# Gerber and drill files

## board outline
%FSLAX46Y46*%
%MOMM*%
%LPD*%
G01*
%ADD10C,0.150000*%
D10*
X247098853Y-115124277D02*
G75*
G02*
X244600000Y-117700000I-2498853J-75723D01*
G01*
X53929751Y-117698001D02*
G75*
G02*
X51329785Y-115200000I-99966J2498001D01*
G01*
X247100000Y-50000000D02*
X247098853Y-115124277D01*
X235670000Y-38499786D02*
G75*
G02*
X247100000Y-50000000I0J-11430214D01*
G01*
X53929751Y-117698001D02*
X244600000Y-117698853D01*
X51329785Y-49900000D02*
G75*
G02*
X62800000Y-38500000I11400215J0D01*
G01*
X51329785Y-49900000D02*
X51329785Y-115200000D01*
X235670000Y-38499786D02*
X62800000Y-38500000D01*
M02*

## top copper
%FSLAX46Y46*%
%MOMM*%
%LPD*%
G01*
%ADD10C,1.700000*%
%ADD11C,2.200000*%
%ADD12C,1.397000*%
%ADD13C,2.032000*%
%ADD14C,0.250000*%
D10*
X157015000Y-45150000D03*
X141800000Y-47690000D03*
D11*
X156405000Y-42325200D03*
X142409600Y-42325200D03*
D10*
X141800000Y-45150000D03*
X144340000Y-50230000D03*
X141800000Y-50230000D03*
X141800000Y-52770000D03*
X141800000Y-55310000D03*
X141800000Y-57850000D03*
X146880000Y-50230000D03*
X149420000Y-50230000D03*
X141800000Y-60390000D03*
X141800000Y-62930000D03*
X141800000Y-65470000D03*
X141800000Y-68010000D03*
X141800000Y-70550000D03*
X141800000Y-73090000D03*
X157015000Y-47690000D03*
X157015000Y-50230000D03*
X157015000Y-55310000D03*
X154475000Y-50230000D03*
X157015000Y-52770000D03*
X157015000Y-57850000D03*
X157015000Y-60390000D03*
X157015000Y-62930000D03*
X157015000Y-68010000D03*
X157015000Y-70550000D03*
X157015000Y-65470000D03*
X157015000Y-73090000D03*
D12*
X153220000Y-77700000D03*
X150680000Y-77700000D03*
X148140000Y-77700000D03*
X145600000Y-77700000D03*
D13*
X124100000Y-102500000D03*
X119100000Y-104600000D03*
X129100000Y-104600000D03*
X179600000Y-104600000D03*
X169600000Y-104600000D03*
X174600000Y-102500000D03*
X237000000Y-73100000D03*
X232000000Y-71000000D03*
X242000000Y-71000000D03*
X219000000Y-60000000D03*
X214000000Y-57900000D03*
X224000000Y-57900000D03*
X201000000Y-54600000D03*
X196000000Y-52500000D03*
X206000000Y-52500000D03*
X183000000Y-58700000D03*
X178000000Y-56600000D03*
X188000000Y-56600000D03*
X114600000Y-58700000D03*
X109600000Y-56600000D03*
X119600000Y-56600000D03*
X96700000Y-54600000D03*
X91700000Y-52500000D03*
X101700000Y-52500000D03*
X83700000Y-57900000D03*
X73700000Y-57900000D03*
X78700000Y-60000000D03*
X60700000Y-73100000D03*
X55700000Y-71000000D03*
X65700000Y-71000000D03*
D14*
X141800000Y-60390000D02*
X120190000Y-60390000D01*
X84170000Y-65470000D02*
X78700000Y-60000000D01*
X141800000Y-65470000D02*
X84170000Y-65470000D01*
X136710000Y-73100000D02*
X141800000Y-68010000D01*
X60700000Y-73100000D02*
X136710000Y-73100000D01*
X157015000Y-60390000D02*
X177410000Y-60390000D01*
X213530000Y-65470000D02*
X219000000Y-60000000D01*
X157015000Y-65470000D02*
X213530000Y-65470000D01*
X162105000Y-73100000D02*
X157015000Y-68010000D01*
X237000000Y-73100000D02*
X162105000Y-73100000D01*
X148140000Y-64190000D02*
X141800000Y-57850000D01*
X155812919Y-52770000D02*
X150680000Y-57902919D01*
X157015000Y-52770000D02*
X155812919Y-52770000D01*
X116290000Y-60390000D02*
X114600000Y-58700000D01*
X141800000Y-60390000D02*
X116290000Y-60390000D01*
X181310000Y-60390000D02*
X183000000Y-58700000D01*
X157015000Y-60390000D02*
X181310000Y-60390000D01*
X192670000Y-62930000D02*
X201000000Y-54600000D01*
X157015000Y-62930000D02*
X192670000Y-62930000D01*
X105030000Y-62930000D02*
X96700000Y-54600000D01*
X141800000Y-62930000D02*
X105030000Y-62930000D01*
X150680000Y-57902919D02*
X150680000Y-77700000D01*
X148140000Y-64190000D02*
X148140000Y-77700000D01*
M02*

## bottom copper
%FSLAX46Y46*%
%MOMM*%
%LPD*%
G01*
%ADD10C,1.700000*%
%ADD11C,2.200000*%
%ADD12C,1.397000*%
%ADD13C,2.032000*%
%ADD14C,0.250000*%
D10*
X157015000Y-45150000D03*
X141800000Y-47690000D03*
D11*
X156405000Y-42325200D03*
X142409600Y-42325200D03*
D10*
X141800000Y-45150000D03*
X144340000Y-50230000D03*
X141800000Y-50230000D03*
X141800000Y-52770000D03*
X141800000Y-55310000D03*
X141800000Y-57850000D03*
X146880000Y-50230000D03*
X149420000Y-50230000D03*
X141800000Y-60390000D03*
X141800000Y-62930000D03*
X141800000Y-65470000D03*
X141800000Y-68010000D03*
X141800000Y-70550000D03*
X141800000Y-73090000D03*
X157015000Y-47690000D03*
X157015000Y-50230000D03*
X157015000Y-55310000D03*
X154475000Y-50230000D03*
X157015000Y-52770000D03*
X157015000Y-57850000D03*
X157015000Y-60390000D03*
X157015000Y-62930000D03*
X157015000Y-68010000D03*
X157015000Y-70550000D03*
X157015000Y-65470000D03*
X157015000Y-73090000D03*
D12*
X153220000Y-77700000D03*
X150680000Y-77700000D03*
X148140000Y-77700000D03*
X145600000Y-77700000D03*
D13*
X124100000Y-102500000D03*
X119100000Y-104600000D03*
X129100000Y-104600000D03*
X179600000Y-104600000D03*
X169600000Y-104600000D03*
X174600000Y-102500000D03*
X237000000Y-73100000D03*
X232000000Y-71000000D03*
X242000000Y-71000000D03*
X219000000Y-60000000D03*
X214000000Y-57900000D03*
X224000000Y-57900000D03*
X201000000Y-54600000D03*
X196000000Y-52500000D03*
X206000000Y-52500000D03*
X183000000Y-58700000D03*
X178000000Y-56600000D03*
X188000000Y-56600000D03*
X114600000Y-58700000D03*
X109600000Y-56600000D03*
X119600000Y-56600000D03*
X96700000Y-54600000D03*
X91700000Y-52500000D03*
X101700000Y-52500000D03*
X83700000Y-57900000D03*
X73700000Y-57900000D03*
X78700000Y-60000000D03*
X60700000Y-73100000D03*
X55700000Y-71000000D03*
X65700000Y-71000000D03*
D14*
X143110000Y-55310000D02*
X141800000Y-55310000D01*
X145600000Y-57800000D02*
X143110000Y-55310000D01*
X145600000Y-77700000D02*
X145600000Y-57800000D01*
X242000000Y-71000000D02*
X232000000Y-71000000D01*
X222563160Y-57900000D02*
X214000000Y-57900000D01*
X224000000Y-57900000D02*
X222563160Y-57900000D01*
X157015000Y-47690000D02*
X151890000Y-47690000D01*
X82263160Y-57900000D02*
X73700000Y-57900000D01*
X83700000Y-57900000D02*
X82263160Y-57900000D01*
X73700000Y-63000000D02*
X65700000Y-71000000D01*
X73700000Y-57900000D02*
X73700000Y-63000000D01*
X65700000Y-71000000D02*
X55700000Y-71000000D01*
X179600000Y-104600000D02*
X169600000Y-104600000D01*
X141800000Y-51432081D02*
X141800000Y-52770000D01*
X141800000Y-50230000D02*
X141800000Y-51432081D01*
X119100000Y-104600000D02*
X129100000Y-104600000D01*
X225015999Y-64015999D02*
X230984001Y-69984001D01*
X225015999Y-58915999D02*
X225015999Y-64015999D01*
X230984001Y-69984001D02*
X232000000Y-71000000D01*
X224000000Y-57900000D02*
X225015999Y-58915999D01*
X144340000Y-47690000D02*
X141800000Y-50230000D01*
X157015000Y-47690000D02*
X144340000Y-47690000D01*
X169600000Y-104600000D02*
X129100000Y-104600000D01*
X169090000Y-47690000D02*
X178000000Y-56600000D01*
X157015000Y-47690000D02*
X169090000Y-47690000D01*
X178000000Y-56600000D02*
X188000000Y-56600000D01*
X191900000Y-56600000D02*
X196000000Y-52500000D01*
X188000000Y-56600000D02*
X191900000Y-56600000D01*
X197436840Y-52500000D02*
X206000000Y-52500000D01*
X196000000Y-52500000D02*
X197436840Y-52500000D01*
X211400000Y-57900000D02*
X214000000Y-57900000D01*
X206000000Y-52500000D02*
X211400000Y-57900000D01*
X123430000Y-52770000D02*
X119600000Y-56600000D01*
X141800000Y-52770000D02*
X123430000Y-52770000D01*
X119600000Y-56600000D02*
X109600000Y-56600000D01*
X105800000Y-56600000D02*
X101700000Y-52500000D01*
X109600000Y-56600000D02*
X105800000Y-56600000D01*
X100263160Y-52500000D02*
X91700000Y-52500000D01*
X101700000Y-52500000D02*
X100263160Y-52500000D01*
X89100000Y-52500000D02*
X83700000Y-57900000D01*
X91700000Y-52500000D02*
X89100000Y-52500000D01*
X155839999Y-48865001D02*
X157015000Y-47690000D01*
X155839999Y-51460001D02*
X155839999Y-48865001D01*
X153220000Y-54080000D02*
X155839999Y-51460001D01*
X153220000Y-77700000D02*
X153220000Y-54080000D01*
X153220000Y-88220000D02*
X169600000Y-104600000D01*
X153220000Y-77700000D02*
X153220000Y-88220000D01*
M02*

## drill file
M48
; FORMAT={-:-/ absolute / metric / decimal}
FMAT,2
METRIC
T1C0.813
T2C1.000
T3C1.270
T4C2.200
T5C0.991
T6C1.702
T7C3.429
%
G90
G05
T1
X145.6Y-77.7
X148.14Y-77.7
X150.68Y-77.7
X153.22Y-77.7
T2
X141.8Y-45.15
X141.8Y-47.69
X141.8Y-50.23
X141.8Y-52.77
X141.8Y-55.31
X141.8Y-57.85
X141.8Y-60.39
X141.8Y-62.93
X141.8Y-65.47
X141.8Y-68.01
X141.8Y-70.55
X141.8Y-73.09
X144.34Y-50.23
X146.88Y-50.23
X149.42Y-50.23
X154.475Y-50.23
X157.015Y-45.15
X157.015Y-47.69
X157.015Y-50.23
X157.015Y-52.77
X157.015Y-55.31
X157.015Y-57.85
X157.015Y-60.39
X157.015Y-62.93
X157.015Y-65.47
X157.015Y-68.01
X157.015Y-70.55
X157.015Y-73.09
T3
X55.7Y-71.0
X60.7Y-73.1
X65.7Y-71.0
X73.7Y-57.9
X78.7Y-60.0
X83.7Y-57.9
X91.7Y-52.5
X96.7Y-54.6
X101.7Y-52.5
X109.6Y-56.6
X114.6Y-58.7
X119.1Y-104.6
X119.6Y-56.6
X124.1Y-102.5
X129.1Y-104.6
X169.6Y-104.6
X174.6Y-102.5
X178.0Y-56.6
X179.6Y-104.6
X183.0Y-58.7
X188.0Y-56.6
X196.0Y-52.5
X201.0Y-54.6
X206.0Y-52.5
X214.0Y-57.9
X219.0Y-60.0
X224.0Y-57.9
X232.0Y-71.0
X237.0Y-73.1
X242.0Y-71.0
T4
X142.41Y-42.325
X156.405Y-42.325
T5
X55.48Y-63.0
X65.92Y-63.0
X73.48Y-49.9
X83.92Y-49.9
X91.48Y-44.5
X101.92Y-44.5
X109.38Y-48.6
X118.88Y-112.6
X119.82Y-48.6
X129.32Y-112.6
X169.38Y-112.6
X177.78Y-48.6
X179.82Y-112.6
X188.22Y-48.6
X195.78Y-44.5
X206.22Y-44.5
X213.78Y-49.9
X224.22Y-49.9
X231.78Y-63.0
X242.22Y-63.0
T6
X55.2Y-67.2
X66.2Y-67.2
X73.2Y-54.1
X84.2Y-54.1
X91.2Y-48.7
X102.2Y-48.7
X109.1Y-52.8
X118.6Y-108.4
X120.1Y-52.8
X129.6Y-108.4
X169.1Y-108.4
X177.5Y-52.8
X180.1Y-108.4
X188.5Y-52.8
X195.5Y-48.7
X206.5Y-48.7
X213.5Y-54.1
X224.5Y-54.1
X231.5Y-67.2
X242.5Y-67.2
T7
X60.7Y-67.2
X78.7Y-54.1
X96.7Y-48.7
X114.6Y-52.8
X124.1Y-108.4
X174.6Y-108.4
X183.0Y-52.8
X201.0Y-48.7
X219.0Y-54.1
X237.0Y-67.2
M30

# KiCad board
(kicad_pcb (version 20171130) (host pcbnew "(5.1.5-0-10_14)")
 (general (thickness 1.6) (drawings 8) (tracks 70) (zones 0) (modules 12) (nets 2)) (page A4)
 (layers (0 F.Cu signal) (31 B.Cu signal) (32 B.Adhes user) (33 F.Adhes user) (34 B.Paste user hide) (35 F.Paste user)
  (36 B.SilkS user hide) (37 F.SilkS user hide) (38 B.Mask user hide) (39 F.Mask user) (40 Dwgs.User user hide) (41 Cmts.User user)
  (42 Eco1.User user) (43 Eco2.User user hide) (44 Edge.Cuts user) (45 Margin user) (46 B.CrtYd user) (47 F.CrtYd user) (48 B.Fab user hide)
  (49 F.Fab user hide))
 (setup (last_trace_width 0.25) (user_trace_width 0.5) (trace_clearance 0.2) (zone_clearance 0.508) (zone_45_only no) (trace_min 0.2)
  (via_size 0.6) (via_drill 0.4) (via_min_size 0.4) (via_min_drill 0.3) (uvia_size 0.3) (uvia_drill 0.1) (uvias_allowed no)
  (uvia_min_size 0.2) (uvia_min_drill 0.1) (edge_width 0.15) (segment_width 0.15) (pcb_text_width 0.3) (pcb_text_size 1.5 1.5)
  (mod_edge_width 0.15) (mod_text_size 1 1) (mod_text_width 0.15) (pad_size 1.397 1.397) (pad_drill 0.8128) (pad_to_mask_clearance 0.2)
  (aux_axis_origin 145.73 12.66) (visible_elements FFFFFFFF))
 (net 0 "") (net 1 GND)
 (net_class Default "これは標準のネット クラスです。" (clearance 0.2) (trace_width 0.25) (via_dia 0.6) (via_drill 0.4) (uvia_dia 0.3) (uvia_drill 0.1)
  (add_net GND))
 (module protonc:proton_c (layer F.Cu) (at 149.4 60.4)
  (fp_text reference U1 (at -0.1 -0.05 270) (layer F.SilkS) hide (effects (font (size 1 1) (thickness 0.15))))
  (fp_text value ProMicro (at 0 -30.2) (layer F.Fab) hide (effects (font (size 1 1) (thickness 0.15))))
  (pad 5V thru_hole circle (at 7.615 -15.25) (size 1.7 1.7) (drill 1) (layers *.Cu *.Mask))
  (pad A10 thru_hole circle (at -7.6 -12.71) (size 1.7 1.7) (drill 1) (layers *.Cu *.Mask))
  (pad SCRE thru_hole circle (at 7.005 -18.0748) (size 2.2 2.2) (drill 2.2) (layers *.Cu *.Mask))
  (pad SCRE thru_hole circle (at -6.9904 -18.0748) (size 2.2 2.2) (drill 2.2) (layers *.Cu *.Mask))
  (pad A9 thru_hole circle (at -7.6 -15.25) (size 1.7 1.7) (drill 1) (layers *.Cu *.Mask))
  (pad D+ thru_hole circle (at -5.06 -10.17) (size 1.7 1.7) (drill 1) (layers *.Cu *.Mask))
  (pad GND thru_hole circle (at -7.6 -10.17) (size 1.7 1.7) (drill 1) (layers *.Cu *.Mask) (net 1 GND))
  (pad GND thru_hole circle (at -7.6 -7.63) (size 1.7 1.7) (drill 1) (layers *.Cu *.Mask) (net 1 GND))
  (pad B7 thru_hole circle (at -7.6 -5.09) (size 1.7 1.7) (drill 1) (layers *.Cu *.Mask))
  (pad B6 thru_hole circle (at -7.6 -2.55) (size 1.7 1.7) (drill 1) (layers *.Cu *.Mask))
  (pad D- thru_hole circle (at -2.52 -10.17) (size 1.7 1.7) (drill 1) (layers *.Cu *.Mask))
  (pad CHRG thru_hole circle (at 0.02 -10.17) (size 1.7 1.7) (drill 1) (layers *.Cu *.Mask))
  (pad B5 thru_hole circle (at -7.6 -0.01) (size 1.7 1.7) (drill 1) (layers *.Cu *.Mask))
  (pad B4 thru_hole circle (at -7.6 2.53) (size 1.7 1.7) (drill 1) (layers *.Cu *.Mask))
  (pad B3 thru_hole circle (at -7.6 5.07) (size 1.7 1.7) (drill 1) (layers *.Cu *.Mask))
  (pad B2 thru_hole circle (at -7.6 7.61) (size 1.7 1.7) (drill 1) (layers *.Cu *.Mask))
  (pad B1 thru_hole circle (at -7.6 10.15) (size 1.7 1.7) (drill 1) (layers *.Cu *.Mask))
  (pad B0 thru_hole circle (at -7.6 12.69) (size 1.7 1.7) (drill 1) (layers *.Cu *.Mask))
  (pad GND thru_hole circle (at 7.615 -12.71) (size 1.7 1.7) (drill 1) (layers *.Cu *.Mask) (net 1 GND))
  (pad DFU thru_hole circle (at 7.615 -10.17) (size 1.7 1.7) (drill 1) (layers *.Cu *.Mask))
  (pad A2 thru_hole circle (at 7.615 -5.09) (size 1.7 1.7) (drill 1) (layers *.Cu *.Mask))
  (pad A3|5v thru_hole circle (at 5.075 -10.17) (size 1.7 1.7) (drill 1) (layers *.Cu *.Mask))
  (pad 3.3V thru_hole circle (at 7.615 -7.63) (size 1.7 1.7) (drill 1) (layers *.Cu *.Mask))
  (pad A1 thru_hole circle (at 7.615 -2.55) (size 1.7 1.7) (drill 1) (layers *.Cu *.Mask))
  (pad A0 thru_hole circle (at 7.615 -0.01) (size 1.7 1.7) (drill 1) (layers *.Cu *.Mask))
  (pad B8 thru_hole circle (at 7.615 2.53) (size 1.7 1.7) (drill 1) (layers *.Cu *.Mask))
  (pad B14 thru_hole circle (at 7.615 7.61) (size 1.7 1.7) (drill 1) (layers *.Cu *.Mask))
  (pad B15 thru_hole circle (at 7.615 10.15) (size 1.7 1.7) (drill 1) (layers *.Cu *.Mask))
  (pad B13 thru_hole circle (at 7.615 5.07) (size 1.7 1.7) (drill 1) (layers *.Cu *.Mask))
  (pad B9 thru_hole circle (at 7.615 12.69) (size 1.7 1.7) (drill 1) (layers *.Cu *.Mask)))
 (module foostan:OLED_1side (layer F.Cu) (at 145.6 77.7)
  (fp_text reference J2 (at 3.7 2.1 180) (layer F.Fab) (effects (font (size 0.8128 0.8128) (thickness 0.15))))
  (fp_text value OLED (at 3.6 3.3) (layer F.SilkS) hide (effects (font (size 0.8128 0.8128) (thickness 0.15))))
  (pad 4 thru_hole circle (at 7.62 0) (size 1.397 1.397) (drill 0.8128) (layers *.Cu F.SilkS B.Mask) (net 1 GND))
  (pad 3 thru_hole circle (at 5.08 0) (size 1.397 1.397) (drill 0.8128) (layers *.Cu F.SilkS B.Mask))
  (pad 2 thru_hole circle (at 2.54 0) (size 1.397 1.397) (drill 0.8128) (layers *.Cu F.SilkS B.Mask))
  (pad 1 thru_hole circle (at 0 0) (size 1.397 1.397) (drill 0.8128) (layers *.Cu F.SilkS B.Mask)))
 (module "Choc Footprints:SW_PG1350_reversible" (layer B.Cu) (at 124.1 108.4)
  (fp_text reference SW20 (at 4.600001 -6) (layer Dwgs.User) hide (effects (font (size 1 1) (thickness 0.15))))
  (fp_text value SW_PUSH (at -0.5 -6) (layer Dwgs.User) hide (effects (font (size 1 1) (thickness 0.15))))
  (pad "" np_thru_hole circle (at -5.5 0) (size 1.7018 1.7018) (drill 1.7018) (layers *.Cu *.Mask))
  (pad "" np_thru_hole circle (at 5.5 0) (size 1.7018 1.7018) (drill 1.7018) (layers *.Cu *.Mask))
  (pad "" np_thru_hole circle (at 5.22 4.2) (size 0.9906 0.9906) (drill 0.9906) (layers *.Cu *.Mask))
  (pad 1 thru_hole circle (at 0 -5.9) (size 2.032 2.032) (drill 1.27) (layers *.Cu *.Mask))
  (pad 2 thru_hole circle (at -5 -3.8) (size 2.032 2.032) (drill 1.27) (layers *.Cu *.Mask) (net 1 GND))
  (pad "" np_thru_hole circle (at 0 0) (size 3.429 3.429) (drill 3.429) (layers *.Cu *.Mask))
  (pad 2 thru_hole circle (at 5 -3.8) (size 2.032 2.032) (drill 1.27) (layers *.Cu *.Mask) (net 1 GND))
  (pad "" np_thru_hole circle (at -5.22 4.2) (size 0.9906 0.9906) (drill 0.9906) (layers *.Cu *.Mask)))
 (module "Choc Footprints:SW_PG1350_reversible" (layer B.Cu) (at 174.6 108.4)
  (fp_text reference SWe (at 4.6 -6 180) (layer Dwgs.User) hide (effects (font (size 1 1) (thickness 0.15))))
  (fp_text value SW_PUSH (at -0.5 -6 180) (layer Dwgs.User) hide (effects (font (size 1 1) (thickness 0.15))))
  (pad "" np_thru_hole circle (at -5.22 4.2) (size 0.9906 0.9906) (drill 0.9906) (layers *.Cu *.Mask))
  (pad 2 thru_hole circle (at 5 -3.8) (size 2.032 2.032) (drill 1.27) (layers *.Cu *.Mask) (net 1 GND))
  (pad "" np_thru_hole circle (at 0 0) (size 3.429 3.429) (drill 3.429) (layers *.Cu *.Mask))
  (pad 2 thru_hole circle (at -5 -3.8) (size 2.032 2.032) (drill 1.27) (layers *.Cu *.Mask) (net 1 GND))
  (pad 1 thru_hole circle (at 0 -5.9) (size 2.032 2.032) (drill 1.27) (layers *.Cu *.Mask))
  (pad "" np_thru_hole circle (at 5.22 4.2) (size 0.9906 0.9906) (drill 0.9906) (layers *.Cu *.Mask))
  (pad "" np_thru_hole circle (at 5.5 0) (size 1.7018 1.7018) (drill 1.7018) (layers *.Cu *.Mask))
  (pad "" np_thru_hole circle (at -5.5 0) (size 1.7018 1.7018) (drill 1.7018) (layers *.Cu *.Mask)))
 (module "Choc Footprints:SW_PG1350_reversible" (layer F.Cu) (at 237 67.2)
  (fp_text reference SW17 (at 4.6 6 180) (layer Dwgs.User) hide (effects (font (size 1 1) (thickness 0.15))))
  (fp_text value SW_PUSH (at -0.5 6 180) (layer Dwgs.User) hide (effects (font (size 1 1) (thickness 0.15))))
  (pad "" np_thru_hole circle (at -5.5 0) (size 1.7018 1.7018) (drill 1.7018) (layers *.Cu *.Mask))
  (pad "" np_thru_hole circle (at 5.5 0) (size 1.7018 1.7018) (drill 1.7018) (layers *.Cu *.Mask))
  (pad "" np_thru_hole circle (at 5.22 -4.2) (size 0.9906 0.9906) (drill 0.9906) (layers *.Cu *.Mask))
  (pad 1 thru_hole circle (at 0 5.9) (size 2.032 2.032) (drill 1.27) (layers *.Cu *.Mask))
  (pad 2 thru_hole circle (at -5 3.8) (size 2.032 2.032) (drill 1.27) (layers *.Cu *.Mask) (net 1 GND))
  (pad "" np_thru_hole circle (at 0 0) (size 3.429 3.429) (drill 3.429) (layers *.Cu *.Mask))
  (pad 2 thru_hole circle (at 5 3.8) (size 2.032 2.032) (drill 1.27) (layers *.Cu *.Mask) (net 1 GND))
  (pad "" np_thru_hole circle (at -5.22 -4.2) (size 0.9906 0.9906) (drill 0.9906) (layers *.Cu *.Mask)))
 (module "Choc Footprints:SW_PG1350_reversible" (layer F.Cu) (at 219 54.1)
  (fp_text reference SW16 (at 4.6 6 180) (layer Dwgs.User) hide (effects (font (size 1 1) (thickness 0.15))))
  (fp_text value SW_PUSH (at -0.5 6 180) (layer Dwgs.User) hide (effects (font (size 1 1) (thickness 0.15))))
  (pad "" np_thru_hole circle (at -5.5 0) (size 1.7018 1.7018) (drill 1.7018) (layers *.Cu *.Mask))
  (pad "" np_thru_hole circle (at 5.5 0) (size 1.7018 1.7018) (drill 1.7018) (layers *.Cu *.Mask))
  (pad "" np_thru_hole circle (at 5.22 -4.2) (size 0.9906 0.9906) (drill 0.9906) (layers *.Cu *.Mask))
  (pad 1 thru_hole circle (at 0 5.9) (size 2.032 2.032) (drill 1.27) (layers *.Cu *.Mask))
  (pad 2 thru_hole circle (at -5 3.8) (size 2.032 2.032) (drill 1.27) (layers *.Cu *.Mask) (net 1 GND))
  (pad "" np_thru_hole circle (at 0 0) (size 3.429 3.429) (drill 3.429) (layers *.Cu *.Mask))
  (pad 2 thru_hole circle (at 5 3.8) (size 2.032 2.032) (drill 1.27) (layers *.Cu *.Mask) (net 1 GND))
  (pad "" np_thru_hole circle (at -5.22 -4.2) (size 0.9906 0.9906) (drill 0.9906) (layers *.Cu *.Mask)))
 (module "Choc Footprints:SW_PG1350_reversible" (layer F.Cu) (at 201 48.7)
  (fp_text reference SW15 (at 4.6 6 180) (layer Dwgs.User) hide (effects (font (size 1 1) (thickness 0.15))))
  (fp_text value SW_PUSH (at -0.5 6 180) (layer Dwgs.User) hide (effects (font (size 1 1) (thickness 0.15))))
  (pad "" np_thru_hole circle (at -5.5 0) (size 1.7018 1.7018) (drill 1.7018) (layers *.Cu *.Mask))
  (pad "" np_thru_hole circle (at 5.5 0) (size 1.7018 1.7018) (drill 1.7018) (layers *.Cu *.Mask))
  (pad "" np_thru_hole circle (at 5.22 -4.2) (size 0.9906 0.9906) (drill 0.9906) (layers *.Cu *.Mask))
  (pad 1 thru_hole circle (at 0 5.9) (size 2.032 2.032) (drill 1.27) (layers *.Cu *.Mask))
  (pad 2 thru_hole circle (at -5 3.8) (size 2.032 2.032) (drill 1.27) (layers *.Cu *.Mask) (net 1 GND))
  (pad "" np_thru_hole circle (at 0 0) (size 3.429 3.429) (drill 3.429) (layers *.Cu *.Mask))
  (pad 2 thru_hole circle (at 5 3.8) (size 2.032 2.032) (drill 1.27) (layers *.Cu *.Mask) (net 1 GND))
  (pad "" np_thru_hole circle (at -5.22 -4.2) (size 0.9906 0.9906) (drill 0.9906) (layers *.Cu *.Mask)))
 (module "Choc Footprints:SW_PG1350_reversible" (layer F.Cu) (at 183 52.8)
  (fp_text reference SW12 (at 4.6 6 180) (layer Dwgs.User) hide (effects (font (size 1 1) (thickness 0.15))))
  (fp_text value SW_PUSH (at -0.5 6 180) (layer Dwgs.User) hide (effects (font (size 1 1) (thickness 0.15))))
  (pad "" np_thru_hole circle (at -5.5 0) (size 1.7018 1.7018) (drill 1.7018) (layers *.Cu *.Mask))
  (pad "" np_thru_hole circle (at 5.5 0) (size 1.7018 1.7018) (drill 1.7018) (layers *.Cu *.Mask))
  (pad "" np_thru_hole circle (at 5.22 -4.2) (size 0.9906 0.9906) (drill 0.9906) (layers *.Cu *.Mask))
  (pad 1 thru_hole circle (at 0 5.9) (size 2.032 2.032) (drill 1.27) (layers *.Cu *.Mask))
  (pad 2 thru_hole circle (at -5 3.8) (size 2.032 2.032) (drill 1.27) (layers *.Cu *.Mask) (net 1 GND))
  (pad "" np_thru_hole circle (at 0 0) (size 3.429 3.429) (drill 3.429) (layers *.Cu *.Mask))
  (pad 2 thru_hole circle (at 5 3.8) (size 2.032 2.032) (drill 1.27) (layers *.Cu *.Mask) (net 1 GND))
  (pad "" np_thru_hole circle (at -5.22 -4.2) (size 0.9906 0.9906) (drill 0.9906) (layers *.Cu *.Mask)))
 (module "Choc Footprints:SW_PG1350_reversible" (layer F.Cu) (at 114.6 52.8)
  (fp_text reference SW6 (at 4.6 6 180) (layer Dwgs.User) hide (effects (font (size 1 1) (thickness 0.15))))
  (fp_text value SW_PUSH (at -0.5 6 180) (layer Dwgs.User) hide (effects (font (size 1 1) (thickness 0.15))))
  (pad "" np_thru_hole circle (at -5.5 0) (size 1.7018 1.7018) (drill 1.7018) (layers *.Cu *.Mask))
  (pad "" np_thru_hole circle (at 5.5 0) (size 1.7018 1.7018) (drill 1.7018) (layers *.Cu *.Mask))
  (pad "" np_thru_hole circle (at 5.22 -4.2) (size 0.9906 0.9906) (drill 0.9906) (layers *.Cu *.Mask))
  (pad 1 thru_hole circle (at 0 5.9) (size 2.032 2.032) (drill 1.27) (layers *.Cu *.Mask))
  (pad 2 thru_hole circle (at -5 3.8) (size 2.032 2.032) (drill 1.27) (layers *.Cu *.Mask) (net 1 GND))
  (pad "" np_thru_hole circle (at 0 0) (size 3.429 3.429) (drill 3.429) (layers *.Cu *.Mask))
  (pad 2 thru_hole circle (at 5 3.8) (size 2.032 2.032) (drill 1.27) (layers *.Cu *.Mask) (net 1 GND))
  (pad "" np_thru_hole circle (at -5.22 -4.2) (size 0.9906 0.9906) (drill 0.9906) (layers *.Cu *.Mask)))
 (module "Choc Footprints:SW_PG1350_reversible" (layer F.Cu) (at 96.7 48.7)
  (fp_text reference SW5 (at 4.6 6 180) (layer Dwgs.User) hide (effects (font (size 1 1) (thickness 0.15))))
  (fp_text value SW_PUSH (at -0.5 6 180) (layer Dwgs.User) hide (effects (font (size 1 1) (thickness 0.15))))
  (pad "" np_thru_hole circle (at -5.5 0) (size 1.7018 1.7018) (drill 1.7018) (layers *.Cu *.Mask))
  (pad "" np_thru_hole circle (at 5.5 0) (size 1.7018 1.7018) (drill 1.7018) (layers *.Cu *.Mask))
  (pad "" np_thru_hole circle (at 5.22 -4.2) (size 0.9906 0.9906) (drill 0.9906) (layers *.Cu *.Mask))
  (pad 1 thru_hole circle (at 0 5.9) (size 2.032 2.032) (drill 1.27) (layers *.Cu *.Mask))
  (pad 2 thru_hole circle (at -5 3.8) (size 2.032 2.032) (drill 1.27) (layers *.Cu *.Mask) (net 1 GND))
  (pad "" np_thru_hole circle (at 0 0) (size 3.429 3.429) (drill 3.429) (layers *.Cu *.Mask))
  (pad 2 thru_hole circle (at 5 3.8) (size 2.032 2.032) (drill 1.27) (layers *.Cu *.Mask) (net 1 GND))
  (pad "" np_thru_hole circle (at -5.22 -4.2) (size 0.9906 0.9906) (drill 0.9906) (layers *.Cu *.Mask)))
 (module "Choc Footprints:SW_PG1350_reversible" (layer F.Cu) (at 78.7 54.1)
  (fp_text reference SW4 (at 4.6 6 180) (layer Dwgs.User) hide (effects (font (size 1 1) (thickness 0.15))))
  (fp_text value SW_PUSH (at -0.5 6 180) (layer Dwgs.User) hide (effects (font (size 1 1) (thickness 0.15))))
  (pad "" np_thru_hole circle (at -5.22 -4.2) (size 0.9906 0.9906) (drill 0.9906) (layers *.Cu *.Mask))
  (pad 2 thru_hole circle (at 5 3.8) (size 2.032 2.032) (drill 1.27) (layers *.Cu *.Mask) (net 1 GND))
  (pad "" np_thru_hole circle (at 0 0) (size 3.429 3.429) (drill 3.429) (layers *.Cu *.Mask))
  (pad 2 thru_hole circle (at -5 3.8) (size 2.032 2.032) (drill 1.27) (layers *.Cu *.Mask) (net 1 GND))
  (pad 1 thru_hole circle (at 0 5.9) (size 2.032 2.032) (drill 1.27) (layers *.Cu *.Mask))
  (pad "" np_thru_hole circle (at 5.22 -4.2) (size 0.9906 0.9906) (drill 0.9906) (layers *.Cu *.Mask))
  (pad "" np_thru_hole circle (at 5.5 0) (size 1.7018 1.7018) (drill 1.7018) (layers *.Cu *.Mask))
  (pad "" np_thru_hole circle (at -5.5 0) (size 1.7018 1.7018) (drill 1.7018) (layers *.Cu *.Mask)))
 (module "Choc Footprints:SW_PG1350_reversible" (layer F.Cu) (at 60.7 67.2)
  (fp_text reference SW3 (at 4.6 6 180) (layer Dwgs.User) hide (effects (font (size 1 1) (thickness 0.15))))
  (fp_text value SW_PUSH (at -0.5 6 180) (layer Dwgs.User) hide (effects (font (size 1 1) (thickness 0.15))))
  (pad "" np_thru_hole circle (at -5.5 0) (size 1.7018 1.7018) (drill 1.7018) (layers *.Cu *.Mask))
  (pad "" np_thru_hole circle (at 5.5 0) (size 1.7018 1.7018) (drill 1.7018) (layers *.Cu *.Mask))
  (pad "" np_thru_hole circle (at 5.22 -4.2) (size 0.9906 0.9906) (drill 0.9906) (layers *.Cu *.Mask))
  (pad 1 thru_hole circle (at 0 5.9) (size 2.032 2.032) (drill 1.27) (layers *.Cu *.Mask))
  (pad 2 thru_hole circle (at -5 3.8) (size 2.032 2.032) (drill 1.27) (layers *.Cu *.Mask) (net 1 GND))
  (pad "" np_thru_hole circle (at 0 0) (size 3.429 3.429) (drill 3.429) (layers *.Cu *.Mask))
  (pad 2 thru_hole circle (at 5 3.8) (size 2.032 2.032) (drill 1.27) (layers *.Cu *.Mask) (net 1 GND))
  (pad "" np_thru_hole circle (at -5.22 -4.2) (size 0.9906 0.9906) (drill 0.9906) (layers *.Cu *.Mask)))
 (gr_arc (start 244.6 115.2) (end 244.6 117.7) (angle -91.73570459) (layer Edge.Cuts) (width 0.15))
 (gr_arc (start 53.829785 115.2) (end 51.329785 115.2) (angle -92.29166034) (layer Edge.Cuts) (width 0.15))
 (gr_line (start 247.1 50) (end 247.098853 115.124277) (angle 90) (layer Edge.Cuts) (width 0.15))
 (gr_arc (start 235.67 49.93) (end 247.1 50) (angle -90.3508884) (layer Edge.Cuts) (width 0.15))
 (gr_line (start 53.929751 117.698001) (end 244.6 117.698853) (angle 90) (layer Edge.Cuts) (width 0.15))
 (gr_arc (start 62.73 49.9) (end 62.8 38.5) (angle -90.35181177) (layer Edge.Cuts) (width 0.15))
 (gr_line (start 51.329785 49.9) (end 51.329785 115.2) (angle 90) (layer Edge.Cuts) (width 0.15))
 (gr_line (start 235.67 38.499786) (end 62.8 38.5) (angle 90) (layer Edge.Cuts) (width 0.15))
 (segment (start 141.8 60.39) (end 120.19 60.39) (width 0.25) (layer F.Cu) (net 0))
 (segment (start 84.17 65.47) (end 78.7 60) (width 0.25) (layer F.Cu) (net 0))
 (segment (start 141.8 65.47) (end 84.17 65.47) (width 0.25) (layer F.Cu) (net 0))
 (segment (start 136.71 73.1) (end 141.8 68.01) (width 0.25) (layer F.Cu) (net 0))
 (segment (start 60.7 73.1) (end 136.71 73.1) (width 0.25) (layer F.Cu) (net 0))
 (segment (start 157.015 60.39) (end 177.41 60.39) (width 0.25) (layer F.Cu) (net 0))
 (segment (start 213.53 65.47) (end 219 60) (width 0.25) (layer F.Cu) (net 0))
 (segment (start 157.015 65.47) (end 213.53 65.47) (width 0.25) (layer F.Cu) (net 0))
 (segment (start 162.105 73.1) (end 157.015 68.01) (width 0.25) (layer F.Cu) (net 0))
 (segment (start 237 73.1) (end 162.105 73.1) (width 0.25) (layer F.Cu) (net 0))
 (segment (start 148.14 64.19) (end 141.8 57.85) (width 0.25) (layer F.Cu) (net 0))
 (segment (start 155.812919 52.77) (end 150.68 57.902919) (width 0.25) (layer F.Cu) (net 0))
 (segment (start 157.015 52.77) (end 155.812919 52.77) (width 0.25) (layer F.Cu) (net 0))
 (segment (start 116.29 60.39) (end 114.6 58.7) (width 0.25) (layer F.Cu) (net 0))
 (segment (start 141.8 60.39) (end 116.29 60.39) (width 0.25) (layer F.Cu) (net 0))
 (segment (start 181.31 60.39) (end 183 58.7) (width 0.25) (layer F.Cu) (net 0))
 (segment (start 157.015 60.39) (end 181.31 60.39) (width 0.25) (layer F.Cu) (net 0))
 (segment (start 192.67 62.93) (end 201 54.6) (width 0.25) (layer F.Cu) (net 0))
 (segment (start 157.015 62.93) (end 192.67 62.93) (width 0.25) (layer F.Cu) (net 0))
 (segment (start 105.03 62.93) (end 96.7 54.6) (width 0.25) (layer F.Cu) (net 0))
 (segment (start 141.8 62.93) (end 105.03 62.93) (width 0.25) (layer F.Cu) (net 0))
 (segment (start 143.11 55.31) (end 141.8 55.31) (width 0.25) (layer B.Cu) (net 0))
 (segment (start 145.6 57.8) (end 143.11 55.31) (width 0.25) (layer B.Cu) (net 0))
 (segment (start 145.6 77.7) (end 145.6 57.8) (width 0.25) (layer B.Cu) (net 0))
 (segment (start 150.68 57.902919) (end 150.68 77.7) (width 0.25) (layer F.Cu) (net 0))
 (segment (start 148.14 64.19) (end 148.14 77.7) (width 0.25) (layer F.Cu) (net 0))
 (segment (start 242 71) (end 232 71) (width 0.25) (layer B.Cu) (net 1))
 (segment (start 222.56316 57.9) (end 214 57.9) (width 0.25) (layer B.Cu) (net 1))
 (segment (start 224 57.9) (end 222.56316 57.9) (width 0.25) (layer B.Cu) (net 1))
 (segment (start 157.015 47.69) (end 151.89 47.69) (width 0.25) (layer B.Cu) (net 1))
 (segment (start 82.26316 57.9) (end 73.7 57.9) (width 0.25) (layer B.Cu) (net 1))
 (segment (start 83.7 57.9) (end 82.26316 57.9) (width 0.25) (layer B.Cu) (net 1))
 (segment (start 73.7 63) (end 65.7 71) (width 0.25) (layer B.Cu) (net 1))
 (segment (start 73.7 57.9) (end 73.7 63) (width 0.25) (layer B.Cu) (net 1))
 (segment (start 65.7 71) (end 55.7 71) (width 0.25) (layer B.Cu) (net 1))
 (segment (start 179.6 104.6) (end 169.6 104.6) (width 0.25) (layer B.Cu) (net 1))
 (segment (start 141.8 51.432081) (end 141.8 52.77) (width 0.25) (layer B.Cu) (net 1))
 (segment (start 141.8 50.23) (end 141.8 51.432081) (width 0.25) (layer B.Cu) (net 1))
 (segment (start 119.1 104.6) (end 129.1 104.6) (width 0.25) (layer B.Cu) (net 1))
 (segment (start 225.015999 64.015999) (end 230.984001 69.984001) (width 0.25) (layer B.Cu) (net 1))
 (segment (start 225.015999 58.915999) (end 225.015999 64.015999) (width 0.25) (layer B.Cu) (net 1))
 (segment (start 230.984001 69.984001) (end 232 71) (width 0.25) (layer B.Cu) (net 1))
 (segment (start 224 57.9) (end 225.015999 58.915999) (width 0.25) (layer B.Cu) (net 1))
 (segment (start 144.34 47.69) (end 141.8 50.23) (width 0.25) (layer B.Cu) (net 1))
 (segment (start 157.015 47.69) (end 144.34 47.69) (width 0.25) (layer B.Cu) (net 1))
 (segment (start 169.6 104.6) (end 129.1 104.6) (width 0.25) (layer B.Cu) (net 1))
 (segment (start 169.09 47.69) (end 178 56.6) (width 0.25) (layer B.Cu) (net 1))
 (segment (start 157.015 47.69) (end 169.09 47.69) (width 0.25) (layer B.Cu) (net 1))
 (segment (start 178 56.6) (end 188 56.6) (width 0.25) (layer B.Cu) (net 1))
 (segment (start 191.9 56.6) (end 196 52.5) (width 0.25) (layer B.Cu) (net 1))
 (segment (start 188 56.6) (end 191.9 56.6) (width 0.25) (layer B.Cu) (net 1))
 (segment (start 197.43684 52.5) (end 206 52.5) (width 0.25) (layer B.Cu) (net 1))
 (segment (start 196 52.5) (end 197.43684 52.5) (width 0.25) (layer B.Cu) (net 1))
 (segment (start 211.4 57.9) (end 214 57.9) (width 0.25) (layer B.Cu) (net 1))
 (segment (start 206 52.5) (end 211.4 57.9) (width 0.25) (layer B.Cu) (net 1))
 (segment (start 123.43 52.77) (end 119.6 56.6) (width 0.25) (layer B.Cu) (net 1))
 (segment (start 141.8 52.77) (end 123.43 52.77) (width 0.25) (layer B.Cu) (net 1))
 (segment (start 119.6 56.6) (end 109.6 56.6) (width 0.25) (layer B.Cu) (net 1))
 (segment (start 105.8 56.6) (end 101.7 52.5) (width 0.25) (layer B.Cu) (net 1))
 (segment (start 109.6 56.6) (end 105.8 56.6) (width 0.25) (layer B.Cu) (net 1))
 (segment (start 100.26316 52.5) (end 91.7 52.5) (width 0.25) (layer B.Cu) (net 1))
 (segment (start 101.7 52.5) (end 100.26316 52.5) (width 0.25) (layer B.Cu) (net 1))
 (segment (start 89.1 52.5) (end 83.7 57.9) (width 0.25) (layer B.Cu) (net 1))
 (segment (start 91.7 52.5) (end 89.1 52.5) (width 0.25) (layer B.Cu) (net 1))
 (segment (start 155.839999 48.865001) (end 157.015 47.69) (width 0.25) (layer B.Cu) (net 1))
 (segment (start 155.839999 51.460001) (end 155.839999 48.865001) (width 0.25) (layer B.Cu) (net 1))
 (segment (start 153.22 54.08) (end 155.839999 51.460001) (width 0.25) (layer B.Cu) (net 1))
 (segment (start 153.22 77.7) (end 153.22 54.08) (width 0.25) (layer B.Cu) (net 1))
 (segment (start 153.22 88.22) (end 169.6 104.6) (width 0.25) (layer B.Cu) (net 1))
 (segment (start 153.22 77.7) (end 153.22 88.22) (width 0.25) (layer B.Cu) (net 1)))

